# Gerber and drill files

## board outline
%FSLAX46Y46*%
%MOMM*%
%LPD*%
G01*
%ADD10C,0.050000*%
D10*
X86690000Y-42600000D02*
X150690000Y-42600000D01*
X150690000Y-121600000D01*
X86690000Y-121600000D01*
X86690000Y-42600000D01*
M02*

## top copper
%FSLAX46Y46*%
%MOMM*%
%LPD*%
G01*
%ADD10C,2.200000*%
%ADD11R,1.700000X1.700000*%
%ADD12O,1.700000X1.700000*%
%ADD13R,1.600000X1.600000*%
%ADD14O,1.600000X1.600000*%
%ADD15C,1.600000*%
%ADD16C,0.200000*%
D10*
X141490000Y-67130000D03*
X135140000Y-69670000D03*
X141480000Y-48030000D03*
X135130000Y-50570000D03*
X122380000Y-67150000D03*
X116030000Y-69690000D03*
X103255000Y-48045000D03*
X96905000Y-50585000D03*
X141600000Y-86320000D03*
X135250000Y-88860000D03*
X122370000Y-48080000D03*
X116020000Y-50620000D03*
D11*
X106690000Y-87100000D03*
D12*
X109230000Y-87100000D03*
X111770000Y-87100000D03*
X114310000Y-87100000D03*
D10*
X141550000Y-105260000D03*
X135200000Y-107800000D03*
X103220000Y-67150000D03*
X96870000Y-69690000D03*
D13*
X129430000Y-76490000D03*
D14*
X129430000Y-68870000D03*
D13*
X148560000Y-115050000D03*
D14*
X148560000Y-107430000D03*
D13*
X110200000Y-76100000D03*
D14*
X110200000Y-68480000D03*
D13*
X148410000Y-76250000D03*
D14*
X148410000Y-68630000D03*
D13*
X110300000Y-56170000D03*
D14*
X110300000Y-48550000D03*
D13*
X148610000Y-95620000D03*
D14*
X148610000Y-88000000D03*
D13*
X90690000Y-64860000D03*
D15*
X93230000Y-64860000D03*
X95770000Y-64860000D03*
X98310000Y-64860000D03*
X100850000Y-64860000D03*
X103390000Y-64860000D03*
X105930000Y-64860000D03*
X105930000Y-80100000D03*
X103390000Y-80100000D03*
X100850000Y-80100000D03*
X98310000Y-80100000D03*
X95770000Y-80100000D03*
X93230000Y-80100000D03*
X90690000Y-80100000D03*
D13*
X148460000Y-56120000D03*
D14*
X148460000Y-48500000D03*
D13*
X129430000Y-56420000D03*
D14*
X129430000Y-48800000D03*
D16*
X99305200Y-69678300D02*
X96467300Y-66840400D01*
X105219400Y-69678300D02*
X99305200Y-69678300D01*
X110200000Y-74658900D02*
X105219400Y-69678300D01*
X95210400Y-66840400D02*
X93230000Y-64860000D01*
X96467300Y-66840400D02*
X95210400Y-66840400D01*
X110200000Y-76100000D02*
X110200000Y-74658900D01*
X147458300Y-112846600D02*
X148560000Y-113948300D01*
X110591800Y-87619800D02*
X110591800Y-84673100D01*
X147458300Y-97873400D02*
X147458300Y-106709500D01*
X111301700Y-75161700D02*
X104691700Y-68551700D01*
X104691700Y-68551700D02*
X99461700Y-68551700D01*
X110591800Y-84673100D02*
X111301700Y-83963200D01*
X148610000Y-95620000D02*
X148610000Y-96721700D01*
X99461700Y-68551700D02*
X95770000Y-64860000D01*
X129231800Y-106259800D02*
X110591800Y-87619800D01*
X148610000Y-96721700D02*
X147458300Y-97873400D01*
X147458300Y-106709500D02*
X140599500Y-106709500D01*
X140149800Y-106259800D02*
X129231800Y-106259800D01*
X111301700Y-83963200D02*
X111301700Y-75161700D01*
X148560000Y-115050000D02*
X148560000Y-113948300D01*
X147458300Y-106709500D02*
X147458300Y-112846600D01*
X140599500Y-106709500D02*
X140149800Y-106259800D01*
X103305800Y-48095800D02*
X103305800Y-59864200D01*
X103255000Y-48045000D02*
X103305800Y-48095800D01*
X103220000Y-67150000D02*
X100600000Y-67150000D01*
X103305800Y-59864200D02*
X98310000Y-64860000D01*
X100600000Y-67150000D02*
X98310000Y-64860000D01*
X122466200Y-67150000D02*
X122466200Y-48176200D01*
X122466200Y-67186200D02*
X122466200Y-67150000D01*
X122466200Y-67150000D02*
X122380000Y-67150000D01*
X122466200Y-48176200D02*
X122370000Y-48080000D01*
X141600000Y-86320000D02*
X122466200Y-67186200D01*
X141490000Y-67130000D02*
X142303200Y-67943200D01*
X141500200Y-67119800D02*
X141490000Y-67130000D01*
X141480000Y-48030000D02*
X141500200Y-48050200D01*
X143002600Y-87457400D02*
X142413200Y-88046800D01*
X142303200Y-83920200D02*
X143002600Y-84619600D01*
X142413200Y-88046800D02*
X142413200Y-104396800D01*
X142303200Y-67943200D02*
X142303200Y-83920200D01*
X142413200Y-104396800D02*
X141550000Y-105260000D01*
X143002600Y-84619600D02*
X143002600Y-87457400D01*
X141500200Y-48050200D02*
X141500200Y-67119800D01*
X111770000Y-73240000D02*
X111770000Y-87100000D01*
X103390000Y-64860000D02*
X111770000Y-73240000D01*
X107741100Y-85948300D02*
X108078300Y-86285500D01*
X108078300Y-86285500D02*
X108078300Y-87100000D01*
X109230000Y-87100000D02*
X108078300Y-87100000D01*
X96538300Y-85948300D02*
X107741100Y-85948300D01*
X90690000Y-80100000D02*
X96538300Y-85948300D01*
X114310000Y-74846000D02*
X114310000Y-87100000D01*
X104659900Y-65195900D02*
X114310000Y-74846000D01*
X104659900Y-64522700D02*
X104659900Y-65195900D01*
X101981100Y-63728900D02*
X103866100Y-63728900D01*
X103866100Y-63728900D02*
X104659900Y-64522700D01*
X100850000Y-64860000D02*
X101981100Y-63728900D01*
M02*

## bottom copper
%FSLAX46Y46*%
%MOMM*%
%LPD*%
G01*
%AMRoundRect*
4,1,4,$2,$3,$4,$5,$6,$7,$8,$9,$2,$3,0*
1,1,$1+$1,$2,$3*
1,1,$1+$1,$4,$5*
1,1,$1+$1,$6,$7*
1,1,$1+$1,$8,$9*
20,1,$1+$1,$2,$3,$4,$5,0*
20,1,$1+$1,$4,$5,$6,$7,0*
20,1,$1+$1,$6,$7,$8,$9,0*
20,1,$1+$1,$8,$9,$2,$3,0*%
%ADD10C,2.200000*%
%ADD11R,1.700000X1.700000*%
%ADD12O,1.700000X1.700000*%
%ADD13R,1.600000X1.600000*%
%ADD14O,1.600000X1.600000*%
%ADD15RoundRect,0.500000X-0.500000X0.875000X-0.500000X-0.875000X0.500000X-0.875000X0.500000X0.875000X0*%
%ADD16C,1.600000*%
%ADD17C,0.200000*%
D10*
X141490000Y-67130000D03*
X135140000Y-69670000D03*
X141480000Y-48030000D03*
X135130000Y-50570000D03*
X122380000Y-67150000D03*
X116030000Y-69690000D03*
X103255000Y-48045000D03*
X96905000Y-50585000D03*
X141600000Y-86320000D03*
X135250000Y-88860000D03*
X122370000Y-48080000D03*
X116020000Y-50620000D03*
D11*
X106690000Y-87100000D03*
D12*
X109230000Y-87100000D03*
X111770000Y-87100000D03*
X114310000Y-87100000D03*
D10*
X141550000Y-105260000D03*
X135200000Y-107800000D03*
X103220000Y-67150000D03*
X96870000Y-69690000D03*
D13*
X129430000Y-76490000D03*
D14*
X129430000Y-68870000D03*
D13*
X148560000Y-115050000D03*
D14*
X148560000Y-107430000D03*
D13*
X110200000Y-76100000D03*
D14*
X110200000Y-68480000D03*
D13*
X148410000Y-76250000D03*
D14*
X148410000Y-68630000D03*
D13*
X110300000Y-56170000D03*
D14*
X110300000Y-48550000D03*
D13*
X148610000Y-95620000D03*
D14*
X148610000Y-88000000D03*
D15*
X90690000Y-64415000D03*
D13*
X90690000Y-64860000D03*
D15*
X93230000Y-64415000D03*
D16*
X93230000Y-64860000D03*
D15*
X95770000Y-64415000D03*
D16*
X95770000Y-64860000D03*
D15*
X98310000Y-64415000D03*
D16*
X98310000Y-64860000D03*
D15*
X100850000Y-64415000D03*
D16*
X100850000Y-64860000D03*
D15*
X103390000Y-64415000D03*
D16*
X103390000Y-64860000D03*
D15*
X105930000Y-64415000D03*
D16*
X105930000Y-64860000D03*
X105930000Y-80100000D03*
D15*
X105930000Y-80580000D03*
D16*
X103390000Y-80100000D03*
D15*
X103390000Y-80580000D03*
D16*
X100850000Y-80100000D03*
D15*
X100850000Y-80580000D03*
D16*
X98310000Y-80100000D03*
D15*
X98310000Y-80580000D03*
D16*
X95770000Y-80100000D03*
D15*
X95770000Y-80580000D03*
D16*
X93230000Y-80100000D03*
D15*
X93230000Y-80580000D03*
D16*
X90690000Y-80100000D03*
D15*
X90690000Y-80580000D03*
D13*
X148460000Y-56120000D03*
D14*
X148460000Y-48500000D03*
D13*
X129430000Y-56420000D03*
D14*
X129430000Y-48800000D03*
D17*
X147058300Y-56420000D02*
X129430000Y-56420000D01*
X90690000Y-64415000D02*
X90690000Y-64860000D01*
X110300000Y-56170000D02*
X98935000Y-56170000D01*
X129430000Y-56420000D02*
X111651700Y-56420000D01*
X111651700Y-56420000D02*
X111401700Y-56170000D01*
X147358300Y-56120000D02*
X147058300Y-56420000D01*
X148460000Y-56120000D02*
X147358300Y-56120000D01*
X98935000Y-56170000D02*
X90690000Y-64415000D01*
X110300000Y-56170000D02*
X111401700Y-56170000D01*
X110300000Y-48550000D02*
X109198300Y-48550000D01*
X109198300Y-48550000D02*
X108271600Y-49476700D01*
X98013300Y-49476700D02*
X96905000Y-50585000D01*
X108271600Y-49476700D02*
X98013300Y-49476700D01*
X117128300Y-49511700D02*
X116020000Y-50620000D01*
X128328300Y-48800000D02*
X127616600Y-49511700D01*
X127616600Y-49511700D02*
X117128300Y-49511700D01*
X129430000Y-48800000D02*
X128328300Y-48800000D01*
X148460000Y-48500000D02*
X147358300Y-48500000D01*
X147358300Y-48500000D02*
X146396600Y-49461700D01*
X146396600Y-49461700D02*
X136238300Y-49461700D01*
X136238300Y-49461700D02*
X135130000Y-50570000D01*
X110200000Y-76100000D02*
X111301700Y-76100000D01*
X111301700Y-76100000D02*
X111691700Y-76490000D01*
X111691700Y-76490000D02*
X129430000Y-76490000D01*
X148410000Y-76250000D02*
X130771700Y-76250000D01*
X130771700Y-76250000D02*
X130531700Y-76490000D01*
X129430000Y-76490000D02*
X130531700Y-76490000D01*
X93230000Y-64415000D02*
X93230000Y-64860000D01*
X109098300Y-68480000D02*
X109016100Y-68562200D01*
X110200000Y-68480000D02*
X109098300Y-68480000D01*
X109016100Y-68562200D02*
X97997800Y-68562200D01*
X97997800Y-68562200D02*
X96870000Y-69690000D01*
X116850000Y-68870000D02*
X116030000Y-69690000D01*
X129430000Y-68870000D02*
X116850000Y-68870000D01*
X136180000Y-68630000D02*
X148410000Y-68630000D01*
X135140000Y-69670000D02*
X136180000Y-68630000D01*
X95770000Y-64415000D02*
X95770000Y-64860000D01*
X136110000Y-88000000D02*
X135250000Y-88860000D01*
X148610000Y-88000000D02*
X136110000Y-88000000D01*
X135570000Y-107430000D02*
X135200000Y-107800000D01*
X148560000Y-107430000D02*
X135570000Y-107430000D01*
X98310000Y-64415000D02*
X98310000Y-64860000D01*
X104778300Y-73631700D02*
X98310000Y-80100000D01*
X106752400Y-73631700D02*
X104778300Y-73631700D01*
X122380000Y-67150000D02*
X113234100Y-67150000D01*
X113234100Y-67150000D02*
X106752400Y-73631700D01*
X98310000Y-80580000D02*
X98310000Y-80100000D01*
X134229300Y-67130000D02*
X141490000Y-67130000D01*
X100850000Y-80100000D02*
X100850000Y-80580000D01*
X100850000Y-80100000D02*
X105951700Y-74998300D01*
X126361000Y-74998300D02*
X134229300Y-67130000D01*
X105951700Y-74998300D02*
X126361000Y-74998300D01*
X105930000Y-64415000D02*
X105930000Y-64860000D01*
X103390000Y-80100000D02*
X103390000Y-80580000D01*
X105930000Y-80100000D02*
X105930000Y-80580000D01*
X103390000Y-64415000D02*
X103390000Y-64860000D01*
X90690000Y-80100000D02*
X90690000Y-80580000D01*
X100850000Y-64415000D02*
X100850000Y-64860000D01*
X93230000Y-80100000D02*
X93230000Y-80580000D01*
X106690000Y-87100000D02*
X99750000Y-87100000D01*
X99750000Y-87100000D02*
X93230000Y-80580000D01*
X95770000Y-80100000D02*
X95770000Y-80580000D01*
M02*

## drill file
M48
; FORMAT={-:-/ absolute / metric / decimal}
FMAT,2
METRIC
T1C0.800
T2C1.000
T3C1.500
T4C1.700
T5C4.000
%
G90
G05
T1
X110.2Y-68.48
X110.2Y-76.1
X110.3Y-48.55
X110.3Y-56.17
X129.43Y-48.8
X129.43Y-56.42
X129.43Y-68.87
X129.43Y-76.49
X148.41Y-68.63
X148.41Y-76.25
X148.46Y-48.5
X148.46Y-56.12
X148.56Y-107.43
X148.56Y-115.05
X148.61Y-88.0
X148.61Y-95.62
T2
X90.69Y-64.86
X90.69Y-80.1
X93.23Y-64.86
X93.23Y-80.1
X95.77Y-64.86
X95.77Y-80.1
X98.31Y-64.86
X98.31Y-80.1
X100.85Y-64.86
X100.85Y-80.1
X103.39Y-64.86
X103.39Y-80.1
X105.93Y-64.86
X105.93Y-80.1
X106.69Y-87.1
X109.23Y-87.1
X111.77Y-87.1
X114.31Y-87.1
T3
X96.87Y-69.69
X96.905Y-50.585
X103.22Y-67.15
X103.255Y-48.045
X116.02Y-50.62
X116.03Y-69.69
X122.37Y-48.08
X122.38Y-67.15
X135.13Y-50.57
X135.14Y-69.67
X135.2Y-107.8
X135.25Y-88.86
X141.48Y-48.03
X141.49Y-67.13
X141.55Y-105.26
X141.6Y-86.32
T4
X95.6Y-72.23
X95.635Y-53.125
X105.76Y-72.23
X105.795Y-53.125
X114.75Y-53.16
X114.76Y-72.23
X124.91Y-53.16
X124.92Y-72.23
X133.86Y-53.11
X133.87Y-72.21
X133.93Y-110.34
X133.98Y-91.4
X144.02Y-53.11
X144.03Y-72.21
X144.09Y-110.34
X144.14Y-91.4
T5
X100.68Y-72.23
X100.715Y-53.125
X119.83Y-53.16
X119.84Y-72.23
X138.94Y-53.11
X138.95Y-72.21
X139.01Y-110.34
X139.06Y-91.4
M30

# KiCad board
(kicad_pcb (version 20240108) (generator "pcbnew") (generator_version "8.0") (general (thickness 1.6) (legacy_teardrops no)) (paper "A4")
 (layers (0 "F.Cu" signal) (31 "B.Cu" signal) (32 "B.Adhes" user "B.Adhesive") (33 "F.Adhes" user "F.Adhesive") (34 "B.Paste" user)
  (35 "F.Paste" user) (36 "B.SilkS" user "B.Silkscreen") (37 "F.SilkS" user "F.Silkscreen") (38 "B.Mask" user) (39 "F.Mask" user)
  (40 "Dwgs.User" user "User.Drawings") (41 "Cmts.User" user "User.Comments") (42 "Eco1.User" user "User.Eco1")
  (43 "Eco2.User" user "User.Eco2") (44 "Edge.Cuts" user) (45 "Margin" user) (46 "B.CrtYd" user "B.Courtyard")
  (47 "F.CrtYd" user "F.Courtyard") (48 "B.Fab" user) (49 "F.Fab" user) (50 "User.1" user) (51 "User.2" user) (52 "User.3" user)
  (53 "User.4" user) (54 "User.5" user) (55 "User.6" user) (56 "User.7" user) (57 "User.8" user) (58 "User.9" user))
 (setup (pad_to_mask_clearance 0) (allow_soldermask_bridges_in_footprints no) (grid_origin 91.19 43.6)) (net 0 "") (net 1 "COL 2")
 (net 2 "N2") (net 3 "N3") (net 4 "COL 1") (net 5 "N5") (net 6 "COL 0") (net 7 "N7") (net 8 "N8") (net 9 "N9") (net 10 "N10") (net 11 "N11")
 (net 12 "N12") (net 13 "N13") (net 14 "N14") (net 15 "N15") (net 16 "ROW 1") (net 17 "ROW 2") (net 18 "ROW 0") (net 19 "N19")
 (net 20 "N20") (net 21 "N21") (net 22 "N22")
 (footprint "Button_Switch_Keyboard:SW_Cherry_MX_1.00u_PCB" (layer "F.Cu") (at 141.49 67.13)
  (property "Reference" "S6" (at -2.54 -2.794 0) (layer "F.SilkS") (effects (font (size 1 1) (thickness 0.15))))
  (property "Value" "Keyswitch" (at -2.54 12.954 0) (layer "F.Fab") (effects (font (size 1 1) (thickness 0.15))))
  (pad "" np_thru_hole circle (at -7.62 5.08) (size 1.7 1.7) (drill 1.7) (layers "*.Cu" "*.Mask"))
  (pad "" np_thru_hole circle (at -2.54 5.08) (size 4 4) (drill 4) (layers "*.Cu" "*.Mask"))
  (pad "" np_thru_hole circle (at 2.54 5.08) (size 1.7 1.7) (drill 1.7) (layers "*.Cu" "*.Mask"))
  (pad "1" thru_hole circle (at 0 0) (size 2.2 2.2) (drill 1.5) (layers "*.Cu" "*.Mask") (remove_unused_layers no) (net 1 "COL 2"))
  (pad "2" thru_hole circle (at -6.35 2.54) (size 2.2 2.2) (drill 1.5) (layers "*.Cu" "*.Mask") (remove_unused_layers no) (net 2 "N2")))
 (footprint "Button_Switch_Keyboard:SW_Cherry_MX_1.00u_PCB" (layer "F.Cu") (at 141.48 48.03)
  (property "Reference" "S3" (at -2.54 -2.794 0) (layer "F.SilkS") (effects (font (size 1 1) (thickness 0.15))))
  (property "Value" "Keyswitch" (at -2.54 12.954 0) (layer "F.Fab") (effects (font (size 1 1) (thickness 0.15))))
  (pad "" np_thru_hole circle (at -7.62 5.08) (size 1.7 1.7) (drill 1.7) (layers "*.Cu" "*.Mask"))
  (pad "" np_thru_hole circle (at -2.54 5.08) (size 4 4) (drill 4) (layers "*.Cu" "*.Mask"))
  (pad "" np_thru_hole circle (at 2.54 5.08) (size 1.7 1.7) (drill 1.7) (layers "*.Cu" "*.Mask"))
  (pad "1" thru_hole circle (at 0 0) (size 2.2 2.2) (drill 1.5) (layers "*.Cu" "*.Mask") (remove_unused_layers no) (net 1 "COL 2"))
  (pad "2" thru_hole circle (at -6.35 2.54) (size 2.2 2.2) (drill 1.5) (layers "*.Cu" "*.Mask") (remove_unused_layers no) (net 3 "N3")))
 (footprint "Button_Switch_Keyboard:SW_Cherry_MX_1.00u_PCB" (layer "F.Cu") (at 122.38 67.15)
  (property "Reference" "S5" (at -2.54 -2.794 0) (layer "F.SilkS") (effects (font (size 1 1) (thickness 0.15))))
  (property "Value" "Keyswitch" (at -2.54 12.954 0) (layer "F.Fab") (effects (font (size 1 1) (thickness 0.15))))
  (pad "" np_thru_hole circle (at -7.62 5.08) (size 1.7 1.7) (drill 1.7) (layers "*.Cu" "*.Mask"))
  (pad "" np_thru_hole circle (at -2.54 5.08) (size 4 4) (drill 4) (layers "*.Cu" "*.Mask"))
  (pad "" np_thru_hole circle (at 2.54 5.08) (size 1.7 1.7) (drill 1.7) (layers "*.Cu" "*.Mask"))
  (pad "1" thru_hole circle (at 0 0) (size 2.2 2.2) (drill 1.5) (layers "*.Cu" "*.Mask") (remove_unused_layers no) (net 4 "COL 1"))
  (pad "2" thru_hole circle (at -6.35 2.54) (size 2.2 2.2) (drill 1.5) (layers "*.Cu" "*.Mask") (remove_unused_layers no) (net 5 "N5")))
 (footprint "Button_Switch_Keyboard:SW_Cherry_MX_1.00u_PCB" (layer "F.Cu") (at 103.255 48.045)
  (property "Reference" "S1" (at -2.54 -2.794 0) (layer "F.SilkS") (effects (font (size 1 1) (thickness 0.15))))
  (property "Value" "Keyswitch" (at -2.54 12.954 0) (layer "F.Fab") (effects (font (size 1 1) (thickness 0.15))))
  (pad "" np_thru_hole circle (at -7.62 5.08) (size 1.7 1.7) (drill 1.7) (layers "*.Cu" "*.Mask"))
  (pad "" np_thru_hole circle (at -2.54 5.08) (size 4 4) (drill 4) (layers "*.Cu" "*.Mask"))
  (pad "" np_thru_hole circle (at 2.54 5.08) (size 1.7 1.7) (drill 1.7) (layers "*.Cu" "*.Mask"))
  (pad "1" thru_hole circle (at 0 0) (size 2.2 2.2) (drill 1.5) (layers "*.Cu" "*.Mask") (remove_unused_layers no) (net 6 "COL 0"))
  (pad "2" thru_hole circle (at -6.35 2.54) (size 2.2 2.2) (drill 1.5) (layers "*.Cu" "*.Mask") (remove_unused_layers no) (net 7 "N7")))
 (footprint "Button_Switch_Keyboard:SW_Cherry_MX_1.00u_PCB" (layer "F.Cu") (at 141.6 86.32)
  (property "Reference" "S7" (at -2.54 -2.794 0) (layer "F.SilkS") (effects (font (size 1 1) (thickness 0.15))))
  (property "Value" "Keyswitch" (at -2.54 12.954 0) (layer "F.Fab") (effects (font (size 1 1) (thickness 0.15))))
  (pad "" np_thru_hole circle (at -7.62 5.08) (size 1.7 1.7) (drill 1.7) (layers "*.Cu" "*.Mask"))
  (pad "" np_thru_hole circle (at -2.54 5.08) (size 4 4) (drill 4) (layers "*.Cu" "*.Mask"))
  (pad "" np_thru_hole circle (at 2.54 5.08) (size 1.7 1.7) (drill 1.7) (layers "*.Cu" "*.Mask"))
  (pad "1" thru_hole circle (at 0 0) (size 2.2 2.2) (drill 1.5) (layers "*.Cu" "*.Mask") (remove_unused_layers no) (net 4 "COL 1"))
  (pad "2" thru_hole circle (at -6.35 2.54) (size 2.2 2.2) (drill 1.5) (layers "*.Cu" "*.Mask") (remove_unused_layers no) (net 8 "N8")))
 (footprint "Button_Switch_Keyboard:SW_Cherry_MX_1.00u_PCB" (layer "F.Cu") (at 122.37 48.08)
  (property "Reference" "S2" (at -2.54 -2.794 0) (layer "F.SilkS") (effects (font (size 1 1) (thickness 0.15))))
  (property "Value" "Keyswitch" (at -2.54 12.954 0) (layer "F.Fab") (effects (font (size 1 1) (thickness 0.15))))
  (pad "" np_thru_hole circle (at -7.62 5.08) (size 1.7 1.7) (drill 1.7) (layers "*.Cu" "*.Mask"))
  (pad "" np_thru_hole circle (at -2.54 5.08) (size 4 4) (drill 4) (layers "*.Cu" "*.Mask"))
  (pad "" np_thru_hole circle (at 2.54 5.08) (size 1.7 1.7) (drill 1.7) (layers "*.Cu" "*.Mask"))
  (pad "1" thru_hole circle (at 0 0) (size 2.2 2.2) (drill 1.5) (layers "*.Cu" "*.Mask") (remove_unused_layers no) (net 4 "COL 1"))
  (pad "2" thru_hole circle (at -6.35 2.54) (size 2.2 2.2) (drill 1.5) (layers "*.Cu" "*.Mask") (remove_unused_layers no) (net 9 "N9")))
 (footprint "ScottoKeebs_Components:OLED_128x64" (layer "F.Cu") (at 110.5 87.1)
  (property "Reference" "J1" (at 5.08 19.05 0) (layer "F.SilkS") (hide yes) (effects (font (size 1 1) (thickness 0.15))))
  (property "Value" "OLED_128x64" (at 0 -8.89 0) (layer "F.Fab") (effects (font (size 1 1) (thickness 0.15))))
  (pad "1" thru_hole rect (at -3.81 0 90) (size 1.7 1.7) (drill 1) (layers "*.Cu" "*.Mask") (remove_unused_layers no) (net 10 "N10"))
  (pad "2" thru_hole oval (at -1.27 0 90) (size 1.7 1.7) (drill 1) (layers "*.Cu" "*.Mask") (remove_unused_layers no) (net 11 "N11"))
  (pad "3" thru_hole oval (at 1.27 0 90) (size 1.7 1.7) (drill 1) (layers "*.Cu" "*.Mask") (remove_unused_layers no) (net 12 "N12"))
  (pad "4" thru_hole oval (at 3.81 0 90) (size 1.7 1.7) (drill 1) (layers "*.Cu" "*.Mask") (remove_unused_layers no) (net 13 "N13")))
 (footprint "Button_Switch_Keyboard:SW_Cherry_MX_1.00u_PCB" (layer "F.Cu") (at 141.55 105.26)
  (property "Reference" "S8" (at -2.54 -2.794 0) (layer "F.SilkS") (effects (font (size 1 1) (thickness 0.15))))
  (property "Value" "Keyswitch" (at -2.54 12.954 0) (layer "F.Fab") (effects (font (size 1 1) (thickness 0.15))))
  (pad "" np_thru_hole circle (at -7.62 5.08) (size 1.7 1.7) (drill 1.7) (layers "*.Cu" "*.Mask"))
  (pad "" np_thru_hole circle (at -2.54 5.08) (size 4 4) (drill 4) (layers "*.Cu" "*.Mask"))
  (pad "" np_thru_hole circle (at 2.54 5.08) (size 1.7 1.7) (drill 1.7) (layers "*.Cu" "*.Mask"))
  (pad "1" thru_hole circle (at 0 0) (size 2.2 2.2) (drill 1.5) (layers "*.Cu" "*.Mask") (remove_unused_layers no) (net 1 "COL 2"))
  (pad "2" thru_hole circle (at -6.35 2.54) (size 2.2 2.2) (drill 1.5) (layers "*.Cu" "*.Mask") (remove_unused_layers no) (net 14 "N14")))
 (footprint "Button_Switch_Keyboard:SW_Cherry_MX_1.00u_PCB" (layer "F.Cu") (at 103.22 67.15)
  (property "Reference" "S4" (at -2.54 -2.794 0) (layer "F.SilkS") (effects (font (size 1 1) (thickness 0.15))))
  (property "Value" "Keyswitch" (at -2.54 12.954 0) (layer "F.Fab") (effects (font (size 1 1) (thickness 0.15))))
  (pad "" np_thru_hole circle (at -7.62 5.08) (size 1.7 1.7) (drill 1.7) (layers "*.Cu" "*.Mask"))
  (pad "" np_thru_hole circle (at -2.54 5.08) (size 4 4) (drill 4) (layers "*.Cu" "*.Mask"))
  (pad "" np_thru_hole circle (at 2.54 5.08) (size 1.7 1.7) (drill 1.7) (layers "*.Cu" "*.Mask"))
  (pad "1" thru_hole circle (at 0 0) (size 2.2 2.2) (drill 1.5) (layers "*.Cu" "*.Mask") (remove_unused_layers no) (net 6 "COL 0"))
  (pad "2" thru_hole circle (at -6.35 2.54) (size 2.2 2.2) (drill 1.5) (layers "*.Cu" "*.Mask") (remove_unused_layers no) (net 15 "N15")))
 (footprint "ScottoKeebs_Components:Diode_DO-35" (layer "B.Cu") (at 129.43 76.49 90)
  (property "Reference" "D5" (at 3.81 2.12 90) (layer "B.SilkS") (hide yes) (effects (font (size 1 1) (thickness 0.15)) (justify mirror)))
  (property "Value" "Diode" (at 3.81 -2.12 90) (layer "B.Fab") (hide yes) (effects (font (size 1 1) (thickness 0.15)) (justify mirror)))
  (pad "1" thru_hole rect (at 0 0 90) (size 1.6 1.6) (drill 0.8) (layers "*.Cu" "*.Mask") (remove_unused_layers no) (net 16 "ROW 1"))
  (pad "2" thru_hole oval (at 7.62 0 90) (size 1.6 1.6) (drill 0.8) (layers "*.Cu" "*.Mask") (remove_unused_layers no) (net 5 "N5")))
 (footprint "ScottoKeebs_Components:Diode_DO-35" (layer "B.Cu") (at 148.56 115.05 90)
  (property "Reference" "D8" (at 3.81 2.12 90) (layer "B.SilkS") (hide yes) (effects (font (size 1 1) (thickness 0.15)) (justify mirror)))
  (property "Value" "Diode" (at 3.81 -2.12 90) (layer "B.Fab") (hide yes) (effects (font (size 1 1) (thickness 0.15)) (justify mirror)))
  (pad "1" thru_hole rect (at 0 0 90) (size 1.6 1.6) (drill 0.8) (layers "*.Cu" "*.Mask") (remove_unused_layers no) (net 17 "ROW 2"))
  (pad "2" thru_hole oval (at 7.62 0 90) (size 1.6 1.6) (drill 0.8) (layers "*.Cu" "*.Mask") (remove_unused_layers no) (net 14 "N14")))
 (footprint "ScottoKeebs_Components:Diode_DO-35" (layer "B.Cu") (at 110.2 76.1 90)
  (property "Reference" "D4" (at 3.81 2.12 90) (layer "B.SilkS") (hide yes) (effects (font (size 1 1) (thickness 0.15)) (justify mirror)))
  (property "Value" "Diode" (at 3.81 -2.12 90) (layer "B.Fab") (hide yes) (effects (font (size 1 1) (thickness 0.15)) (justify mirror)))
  (pad "1" thru_hole rect (at 0 0 90) (size 1.6 1.6) (drill 0.8) (layers "*.Cu" "*.Mask") (remove_unused_layers no) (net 16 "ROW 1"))
  (pad "2" thru_hole oval (at 7.62 0 90) (size 1.6 1.6) (drill 0.8) (layers "*.Cu" "*.Mask") (remove_unused_layers no) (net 15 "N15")))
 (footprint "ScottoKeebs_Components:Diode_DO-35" (layer "B.Cu") (at 148.41 76.25 90)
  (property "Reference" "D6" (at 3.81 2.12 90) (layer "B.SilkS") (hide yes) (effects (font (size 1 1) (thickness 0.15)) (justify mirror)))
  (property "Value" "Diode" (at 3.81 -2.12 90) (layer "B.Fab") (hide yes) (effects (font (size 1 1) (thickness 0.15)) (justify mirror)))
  (pad "1" thru_hole rect (at 0 0 90) (size 1.6 1.6) (drill 0.8) (layers "*.Cu" "*.Mask") (remove_unused_layers no) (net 16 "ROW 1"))
  (pad "2" thru_hole oval (at 7.62 0 90) (size 1.6 1.6) (drill 0.8) (layers "*.Cu" "*.Mask") (remove_unused_layers no) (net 2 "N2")))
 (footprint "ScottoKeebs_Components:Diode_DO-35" (layer "B.Cu") (at 110.3 56.17 90)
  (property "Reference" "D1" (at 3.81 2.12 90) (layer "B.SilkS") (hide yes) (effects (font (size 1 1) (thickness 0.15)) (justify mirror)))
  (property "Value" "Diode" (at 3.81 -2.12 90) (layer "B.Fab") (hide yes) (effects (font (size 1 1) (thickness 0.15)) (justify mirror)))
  (pad "1" thru_hole rect (at 0 0 90) (size 1.6 1.6) (drill 0.8) (layers "*.Cu" "*.Mask") (remove_unused_layers no) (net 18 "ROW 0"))
  (pad "2" thru_hole oval (at 7.62 0 90) (size 1.6 1.6) (drill 0.8) (layers "*.Cu" "*.Mask") (remove_unused_layers no) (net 7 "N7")))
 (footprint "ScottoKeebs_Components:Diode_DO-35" (layer "B.Cu") (at 148.61 95.62 90)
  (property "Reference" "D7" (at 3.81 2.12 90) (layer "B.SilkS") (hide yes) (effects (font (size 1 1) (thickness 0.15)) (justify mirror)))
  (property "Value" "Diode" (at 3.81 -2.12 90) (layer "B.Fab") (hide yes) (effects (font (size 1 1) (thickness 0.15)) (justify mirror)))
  (pad "1" thru_hole rect (at 0 0 90) (size 1.6 1.6) (drill 0.8) (layers "*.Cu" "*.Mask") (remove_unused_layers no) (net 17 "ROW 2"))
  (pad "2" thru_hole oval (at 7.62 0 90) (size 1.6 1.6) (drill 0.8) (layers "*.Cu" "*.Mask") (remove_unused_layers no) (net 8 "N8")))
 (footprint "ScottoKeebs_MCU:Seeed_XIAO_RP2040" (layer "B.Cu") (at 98.31 72.48 -90)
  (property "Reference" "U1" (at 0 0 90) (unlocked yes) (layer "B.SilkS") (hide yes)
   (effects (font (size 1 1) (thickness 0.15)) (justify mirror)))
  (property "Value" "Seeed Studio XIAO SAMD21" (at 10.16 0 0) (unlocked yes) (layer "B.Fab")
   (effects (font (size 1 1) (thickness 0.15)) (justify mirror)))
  (pad "1" smd roundrect (at -8.065 7.62 270) (size 2.75 2) (layers "B.Cu" "B.Paste" "B.Mask") (roundrect_rratio 0.25) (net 18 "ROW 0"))
  (pad "1" thru_hole rect (at -7.62 7.62 180) (size 1.6 1.6) (drill 1) (layers "*.Cu" "*.Mask") (remove_unused_layers no) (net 18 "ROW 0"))
  (pad "2" smd roundrect (at -8.065 5.08 270) (size 2.75 2) (layers "B.Cu" "B.Paste" "B.Mask") (roundrect_rratio 0.25) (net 16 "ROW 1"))
  (pad "2" thru_hole circle (at -7.62 5.08 180) (size 1.6 1.6) (drill 1) (layers "*.Cu" "*.Mask") (remove_unused_layers no) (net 16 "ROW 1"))
  (pad "3" smd roundrect (at -8.065 2.54 270) (size 2.75 2) (layers "B.Cu" "B.Paste" "B.Mask") (roundrect_rratio 0.25) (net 17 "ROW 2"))
  (pad "3" thru_hole circle (at -7.62 2.54 180) (size 1.6 1.6) (drill 1) (layers "*.Cu" "*.Mask") (remove_unused_layers no) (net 17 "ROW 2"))
  (pad "4" smd roundrect (at -8.065 0 270) (size 2.75 2) (layers "B.Cu" "B.Paste" "B.Mask") (roundrect_rratio 0.25) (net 6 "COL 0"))
  (pad "4" thru_hole circle (at -7.62 0 180) (size 1.6 1.6) (drill 1) (layers "*.Cu" "*.Mask") (remove_unused_layers no) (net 6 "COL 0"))
  (pad "5" smd roundrect (at -8.065 -2.54 270) (size 2.75 2) (layers "B.Cu" "B.Paste" "B.Mask") (roundrect_rratio 0.25) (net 13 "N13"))
  (pad "5" thru_hole circle (at -7.62 -2.54 180) (size 1.6 1.6) (drill 1) (layers "*.Cu" "*.Mask") (remove_unused_layers no) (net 13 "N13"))
  (pad "6" smd roundrect (at -8.065 -5.08 270) (size 2.75 2) (layers "B.Cu" "B.Paste" "B.Mask") (roundrect_rratio 0.25) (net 12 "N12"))
  (pad "6" thru_hole circle (at -7.62 -5.08 180) (size 1.6 1.6) (drill 1) (layers "*.Cu" "*.Mask") (remove_unused_layers no) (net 12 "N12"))
  (pad "7" smd roundrect (at -8.065 -7.62 270) (size 2.75 2) (layers "B.Cu" "B.Paste" "B.Mask") (roundrect_rratio 0.25) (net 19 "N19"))
  (pad "7" thru_hole circle (at -7.62 -7.62 180) (size 1.6 1.6) (drill 1) (layers "*.Cu" "*.Mask") (remove_unused_layers no) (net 19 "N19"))
  (pad "8" thru_hole circle (at 7.62 -7.62 180) (size 1.6 1.6) (drill 1) (layers "*.Cu" "*.Mask") (remove_unused_layers no) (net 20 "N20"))
  (pad "8" smd roundrect (at 8.1 -7.62 270) (size 2.75 2) (layers "B.Cu" "B.Paste" "B.Mask") (roundrect_rratio 0.25) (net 20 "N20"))
  (pad "9" thru_hole circle (at 7.62 -5.08 180) (size 1.6 1.6) (drill 1) (layers "*.Cu" "*.Mask") (remove_unused_layers no) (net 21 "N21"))
  (pad "9" smd roundrect (at 8.1 -5.08 270) (size 2.75 2) (layers "B.Cu" "B.Paste" "B.Mask") (roundrect_rratio 0.25) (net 21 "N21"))
  (pad "10" thru_hole circle (at 7.62 -2.54 180) (size 1.6 1.6) (drill 1) (layers "*.Cu" "*.Mask") (remove_unused_layers no) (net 1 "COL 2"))
  (pad "10" smd roundrect (at 8.1 -2.54 270) (size 2.75 2) (layers "B.Cu" "B.Paste" "B.Mask") (roundrect_rratio 0.25) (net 1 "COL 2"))
  (pad "11" thru_hole circle (at 7.62 0 180) (size 1.6 1.6) (drill 1) (layers "*.Cu" "*.Mask") (remove_unused_layers no) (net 4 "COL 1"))
  (pad "11" smd roundrect (at 8.1 0 270) (size 2.75 2) (layers "B.Cu" "B.Paste" "B.Mask") (roundrect_rratio 0.25) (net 4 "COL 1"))
  (pad "12" thru_hole circle (at 7.62 2.54 180) (size 1.6 1.6) (drill 1) (layers "*.Cu" "*.Mask") (remove_unused_layers no) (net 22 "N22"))
  (pad "12" smd roundrect (at 8.1 2.54 270) (size 2.75 2) (layers "B.Cu" "B.Paste" "B.Mask") (roundrect_rratio 0.25) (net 22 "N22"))
  (pad "13" thru_hole circle (at 7.62 5.08 180) (size 1.6 1.6) (drill 1) (layers "*.Cu" "*.Mask") (remove_unused_layers no) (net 10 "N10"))
  (pad "13" smd roundrect (at 8.1 5.08 270) (size 2.75 2) (layers "B.Cu" "B.Paste" "B.Mask") (roundrect_rratio 0.25) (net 10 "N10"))
  (pad "14" thru_hole circle (at 7.62 7.62 180) (size 1.6 1.6) (drill 1) (layers "*.Cu" "*.Mask") (remove_unused_layers no) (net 11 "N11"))
  (pad "14" smd roundrect (at 8.1 7.62 270) (size 2.75 2) (layers "B.Cu" "B.Paste" "B.Mask") (roundrect_rratio 0.25) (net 11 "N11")))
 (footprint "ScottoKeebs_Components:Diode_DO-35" (layer "B.Cu") (at 148.46 56.12 90)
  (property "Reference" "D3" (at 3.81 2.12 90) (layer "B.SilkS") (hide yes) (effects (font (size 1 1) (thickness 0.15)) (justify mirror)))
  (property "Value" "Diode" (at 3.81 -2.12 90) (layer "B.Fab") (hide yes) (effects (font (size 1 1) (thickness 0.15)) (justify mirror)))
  (pad "1" thru_hole rect (at 0 0 90) (size 1.6 1.6) (drill 0.8) (layers "*.Cu" "*.Mask") (remove_unused_layers no) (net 18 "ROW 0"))
  (pad "2" thru_hole oval (at 7.62 0 90) (size 1.6 1.6) (drill 0.8) (layers "*.Cu" "*.Mask") (remove_unused_layers no) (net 3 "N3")))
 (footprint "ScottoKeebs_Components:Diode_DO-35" (layer "B.Cu") (at 129.43 56.42 90)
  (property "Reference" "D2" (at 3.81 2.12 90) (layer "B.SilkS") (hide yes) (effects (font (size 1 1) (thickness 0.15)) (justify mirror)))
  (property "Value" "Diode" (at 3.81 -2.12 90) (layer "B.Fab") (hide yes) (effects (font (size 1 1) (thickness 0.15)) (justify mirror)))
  (pad "1" thru_hole rect (at 0 0 90) (size 1.6 1.6) (drill 0.8) (layers "*.Cu" "*.Mask") (remove_unused_layers no) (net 18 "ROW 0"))
  (pad "2" thru_hole oval (at 7.62 0 90) (size 1.6 1.6) (drill 0.8) (layers "*.Cu" "*.Mask") (remove_unused_layers no) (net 9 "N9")))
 (gr_rect (start 86.69 42.6) (end 150.69 121.6) (stroke (width 0.05) (type default)) (fill none) (layer "Edge.Cuts"))
 (segment (start 147.0583 56.42) (end 129.43 56.42) (width 0.2) (layer "B.Cu") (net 18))
 (segment (start 90.69 64.415) (end 90.69 64.86) (width 0.2) (layer "B.Cu") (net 18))
 (segment (start 110.3 56.17) (end 98.935 56.17) (width 0.2) (layer "B.Cu") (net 18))
 (segment (start 129.43 56.42) (end 111.6517 56.42) (width 0.2) (layer "B.Cu") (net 18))
 (segment (start 111.6517 56.42) (end 111.4017 56.17) (width 0.2) (layer "B.Cu") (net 18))
 (segment (start 147.3583 56.12) (end 147.0583 56.42) (width 0.2) (layer "B.Cu") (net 18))
 (segment (start 148.46 56.12) (end 147.3583 56.12) (width 0.2) (layer "B.Cu") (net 18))
 (segment (start 98.935 56.17) (end 90.69 64.415) (width 0.2) (layer "B.Cu") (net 18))
 (segment (start 110.3 56.17) (end 111.4017 56.17) (width 0.2) (layer "B.Cu") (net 18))
 (segment (start 110.3 48.55) (end 109.1983 48.55) (width 0.2) (layer "B.Cu") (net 7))
 (segment (start 109.1983 48.55) (end 108.2716 49.4767) (width 0.2) (layer "B.Cu") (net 7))
 (segment (start 98.0133 49.4767) (end 96.905 50.585) (width 0.2) (layer "B.Cu") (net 7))
 (segment (start 108.2716 49.4767) (end 98.0133 49.4767) (width 0.2) (layer "B.Cu") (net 7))
 (segment (start 117.1283 49.5117) (end 116.02 50.62) (width 0.2) (layer "B.Cu") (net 9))
 (segment (start 128.3283 48.8) (end 127.6166 49.5117) (width 0.2) (layer "B.Cu") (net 9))
 (segment (start 127.6166 49.5117) (end 117.1283 49.5117) (width 0.2) (layer "B.Cu") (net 9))
 (segment (start 129.43 48.8) (end 128.3283 48.8) (width 0.2) (layer "B.Cu") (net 9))
 (segment (start 148.46 48.5) (end 147.3583 48.5) (width 0.2) (layer "B.Cu") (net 3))
 (segment (start 147.3583 48.5) (end 146.3966 49.4617) (width 0.2) (layer "B.Cu") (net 3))
 (segment (start 146.3966 49.4617) (end 136.2383 49.4617) (width 0.2) (layer "B.Cu") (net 3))
 (segment (start 136.2383 49.4617) (end 135.13 50.57) (width 0.2) (layer "B.Cu") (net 3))
 (segment (start 99.3052 69.6783) (end 96.4673 66.8404) (width 0.2) (layer "F.Cu") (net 16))
 (segment (start 105.2194 69.6783) (end 99.3052 69.6783) (width 0.2) (layer "F.Cu") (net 16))
 (segment (start 110.2 74.6589) (end 105.2194 69.6783) (width 0.2) (layer "F.Cu") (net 16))
 (segment (start 95.2104 66.8404) (end 93.23 64.86) (width 0.2) (layer "F.Cu") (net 16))
 (segment (start 96.4673 66.8404) (end 95.2104 66.8404) (width 0.2) (layer "F.Cu") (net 16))
 (segment (start 110.2 76.1) (end 110.2 74.6589) (width 0.2) (layer "F.Cu") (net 16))
 (segment (start 110.2 76.1) (end 111.3017 76.1) (width 0.2) (layer "B.Cu") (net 16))
 (segment (start 111.3017 76.1) (end 111.6917 76.49) (width 0.2) (layer "B.Cu") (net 16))
 (segment (start 111.6917 76.49) (end 129.43 76.49) (width 0.2) (layer "B.Cu") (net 16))
 (segment (start 148.41 76.25) (end 130.7717 76.25) (width 0.2) (layer "B.Cu") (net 16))
 (segment (start 130.7717 76.25) (end 130.5317 76.49) (width 0.2) (layer "B.Cu") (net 16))
 (segment (start 129.43 76.49) (end 130.5317 76.49) (width 0.2) (layer "B.Cu") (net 16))
 (segment (start 93.23 64.415) (end 93.23 64.86) (width 0.2) (layer "B.Cu") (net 16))
 (segment (start 109.0983 68.48) (end 109.0161 68.5622) (width 0.2) (layer "B.Cu") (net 15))
 (segment (start 110.2 68.48) (end 109.0983 68.48) (width 0.2) (layer "B.Cu") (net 15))
 (segment (start 109.0161 68.5622) (end 97.9978 68.5622) (width 0.2) (layer "B.Cu") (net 15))
 (segment (start 97.9978 68.5622) (end 96.87 69.69) (width 0.2) (layer "B.Cu") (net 15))
 (segment (start 116.85 68.87) (end 116.03 69.69) (width 0.2) (layer "B.Cu") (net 5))
 (segment (start 129.43 68.87) (end 116.85 68.87) (width 0.2) (layer "B.Cu") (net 5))
 (segment (start 136.18 68.63) (end 148.41 68.63) (width 0.2) (layer "B.Cu") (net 2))
 (segment (start 135.14 69.67) (end 136.18 68.63) (width 0.2) (layer "B.Cu") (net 2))
 (segment (start 147.4583 112.8466) (end 148.56 113.9483) (width 0.2) (layer "F.Cu") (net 17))
 (segment (start 110.5918 87.6198) (end 110.5918 84.6731) (width 0.2) (layer "F.Cu") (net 17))
 (segment (start 147.4583 97.8734) (end 147.4583 106.7095) (width 0.2) (layer "F.Cu") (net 17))
 (segment (start 111.3017 75.1617) (end 104.6917 68.5517) (width 0.2) (layer "F.Cu") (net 17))
 (segment (start 104.6917 68.5517) (end 99.4617 68.5517) (width 0.2) (layer "F.Cu") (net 17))
 (segment (start 110.5918 84.6731) (end 111.3017 83.9632) (width 0.2) (layer "F.Cu") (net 17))
 (segment (start 148.61 95.62) (end 148.61 96.7217) (width 0.2) (layer "F.Cu") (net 17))
 (segment (start 99.4617 68.5517) (end 95.77 64.86) (width 0.2) (layer "F.Cu") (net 17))
 (segment (start 129.2318 106.2598) (end 110.5918 87.6198) (width 0.2) (layer "F.Cu") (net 17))
 (segment (start 148.61 96.7217) (end 147.4583 97.8734) (width 0.2) (layer "F.Cu") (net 17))
 (segment (start 147.4583 106.7095) (end 140.5995 106.7095) (width 0.2) (layer "F.Cu") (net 17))
 (segment (start 140.1498 106.2598) (end 129.2318 106.2598) (width 0.2) (layer "F.Cu") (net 17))
 (segment (start 111.3017 83.9632) (end 111.3017 75.1617) (width 0.2) (layer "F.Cu") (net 17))
 (segment (start 148.56 115.05) (end 148.56 113.9483) (width 0.2) (layer "F.Cu") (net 17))
 (segment (start 147.4583 106.7095) (end 147.4583 112.8466) (width 0.2) (layer "F.Cu") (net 17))
 (segment (start 140.5995 106.7095) (end 140.1498 106.2598) (width 0.2) (layer "F.Cu") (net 17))
 (segment (start 95.77 64.415) (end 95.77 64.86) (width 0.2) (layer "B.Cu") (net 17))
 (segment (start 136.11 88) (end 135.25 88.86) (width 0.2) (layer "B.Cu") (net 8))
 (segment (start 148.61 88) (end 136.11 88) (width 0.2) (layer "B.Cu") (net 8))
 (segment (start 135.57 107.43) (end 135.2 107.8) (width 0.2) (layer "B.Cu") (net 14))
 (segment (start 148.56 107.43) (end 135.57 107.43) (width 0.2) (layer "B.Cu") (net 14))
 (segment (start 103.3058 48.0958) (end 103.3058 59.8642) (width 0.2) (layer "F.Cu") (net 6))
 (segment (start 103.255 48.045) (end 103.3058 48.0958) (width 0.2) (layer "F.Cu") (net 6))
 (segment (start 103.22 67.15) (end 100.6 67.15) (width 0.2) (layer "F.Cu") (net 6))
 (segment (start 103.3058 59.8642) (end 98.31 64.86) (width 0.2) (layer "F.Cu") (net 6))
 (segment (start 100.6 67.15) (end 98.31 64.86) (width 0.2) (layer "F.Cu") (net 6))
 (segment (start 98.31 64.415) (end 98.31 64.86) (width 0.2) (layer "B.Cu") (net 6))
 (segment (start 122.4662 67.15) (end 122.4662 48.1762) (width 0.2) (layer "F.Cu") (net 4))
 (segment (start 122.4662 67.1862) (end 122.4662 67.15) (width 0.2) (layer "F.Cu") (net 4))
 (segment (start 122.4662 67.15) (end 122.38 67.15) (width 0.2) (layer "F.Cu") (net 4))
 (segment (start 122.4662 48.1762) (end 122.37 48.08) (width 0.2) (layer "F.Cu") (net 4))
 (segment (start 141.6 86.32) (end 122.4662 67.1862) (width 0.2) (layer "F.Cu") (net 4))
 (segment (start 104.7783 73.6317) (end 98.31 80.1) (width 0.2) (layer "B.Cu") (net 4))
 (segment (start 106.7524 73.6317) (end 104.7783 73.6317) (width 0.2) (layer "B.Cu") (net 4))
 (segment (start 122.38 67.15) (end 113.2341 67.15) (width 0.2) (layer "B.Cu") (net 4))
 (segment (start 113.2341 67.15) (end 106.7524 73.6317) (width 0.2) (layer "B.Cu") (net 4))
 (segment (start 98.31 80.58) (end 98.31 80.1) (width 0.2) (layer "B.Cu") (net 4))
 (segment (start 141.49 67.13) (end 142.3032 67.9432) (width 0.2) (layer "F.Cu") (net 1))
 (segment (start 141.5002 67.1198) (end 141.49 67.13) (width 0.2) (layer "F.Cu") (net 1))
 (segment (start 141.48 48.03) (end 141.5002 48.0502) (width 0.2) (layer "F.Cu") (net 1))
 (segment (start 143.0026 87.4574) (end 142.4132 88.0468) (width 0.2) (layer "F.Cu") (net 1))
 (segment (start 142.3032 83.9202) (end 143.0026 84.6196) (width 0.2) (layer "F.Cu") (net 1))
 (segment (start 142.4132 88.0468) (end 142.4132 104.3968) (width 0.2) (layer "F.Cu") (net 1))
 (segment (start 142.3032 67.9432) (end 142.3032 83.9202) (width 0.2) (layer "F.Cu") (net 1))
 (segment (start 142.4132 104.3968) (end 141.55 105.26) (width 0.2) (layer "F.Cu") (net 1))
 (segment (start 143.0026 84.6196) (end 143.0026 87.4574) (width 0.2) (layer "F.Cu") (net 1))
 (segment (start 141.5002 48.0502) (end 141.5002 67.1198) (width 0.2) (layer "F.Cu") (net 1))
 (segment (start 134.2293 67.13) (end 141.49 67.13) (width 0.2) (layer "B.Cu") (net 1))
 (segment (start 100.85 80.1) (end 100.85 80.58) (width 0.2) (layer "B.Cu") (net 1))
 (segment (start 100.85 80.1) (end 105.9517 74.9983) (width 0.2) (layer "B.Cu") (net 1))
 (segment (start 126.361 74.9983) (end 134.2293 67.13) (width 0.2) (layer "B.Cu") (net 1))
 (segment (start 105.9517 74.9983) (end 126.361 74.9983) (width 0.2) (layer "B.Cu") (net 1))
 (segment (start 105.93 64.415) (end 105.93 64.86) (width 0.2) (layer "B.Cu") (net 19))
 (segment (start 103.39 80.1) (end 103.39 80.58) (width 0.2) (layer "B.Cu") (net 21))
 (segment (start 105.93 80.1) (end 105.93 80.58) (width 0.2) (layer "B.Cu") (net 20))
 (segment (start 111.77 73.24) (end 111.77 87.1) (width 0.2) (layer "F.Cu") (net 12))
 (segment (start 103.39 64.86) (end 111.77 73.24) (width 0.2) (layer "F.Cu") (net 12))
 (segment (start 103.39 64.415) (end 103.39 64.86) (width 0.2) (layer "B.Cu") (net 12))
 (segment (start 107.7411 85.9483) (end 108.0783 86.2855) (width 0.2) (layer "F.Cu") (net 11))
 (segment (start 108.0783 86.2855) (end 108.0783 87.1) (width 0.2) (layer "F.Cu") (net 11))
 (segment (start 109.23 87.1) (end 108.0783 87.1) (width 0.2) (layer "F.Cu") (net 11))
 (segment (start 96.5383 85.9483) (end 107.7411 85.9483) (width 0.2) (layer "F.Cu") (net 11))
 (segment (start 90.69 80.1) (end 96.5383 85.9483) (width 0.2) (layer "F.Cu") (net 11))
 (segment (start 90.69 80.1) (end 90.69 80.58) (width 0.2) (layer "B.Cu") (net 11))
 (segment (start 114.31 74.846) (end 114.31 87.1) (width 0.2) (layer "F.Cu") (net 13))
 (segment (start 104.6599 65.1959) (end 114.31 74.846) (width 0.2) (layer "F.Cu") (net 13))
 (segment (start 104.6599 64.5227) (end 104.6599 65.1959) (width 0.2) (layer "F.Cu") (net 13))
 (segment (start 101.9811 63.7289) (end 103.8661 63.7289) (width 0.2) (layer "F.Cu") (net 13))
 (segment (start 103.8661 63.7289) (end 104.6599 64.5227) (width 0.2) (layer "F.Cu") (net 13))
 (segment (start 100.85 64.86) (end 101.9811 63.7289) (width 0.2) (layer "F.Cu") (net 13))
 (segment (start 100.85 64.415) (end 100.85 64.86) (width 0.2) (layer "B.Cu") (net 13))
 (segment (start 93.23 80.1) (end 93.23 80.58) (width 0.2) (layer "B.Cu") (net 10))
 (segment (start 106.69 87.1) (end 99.75 87.1) (width 0.2) (layer "B.Cu") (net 10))
 (segment (start 99.75 87.1) (end 93.23 80.58) (width 0.2) (layer "B.Cu") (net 10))
 (segment (start 95.77 80.1) (end 95.77 80.58) (width 0.2) (layer "B.Cu") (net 22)))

